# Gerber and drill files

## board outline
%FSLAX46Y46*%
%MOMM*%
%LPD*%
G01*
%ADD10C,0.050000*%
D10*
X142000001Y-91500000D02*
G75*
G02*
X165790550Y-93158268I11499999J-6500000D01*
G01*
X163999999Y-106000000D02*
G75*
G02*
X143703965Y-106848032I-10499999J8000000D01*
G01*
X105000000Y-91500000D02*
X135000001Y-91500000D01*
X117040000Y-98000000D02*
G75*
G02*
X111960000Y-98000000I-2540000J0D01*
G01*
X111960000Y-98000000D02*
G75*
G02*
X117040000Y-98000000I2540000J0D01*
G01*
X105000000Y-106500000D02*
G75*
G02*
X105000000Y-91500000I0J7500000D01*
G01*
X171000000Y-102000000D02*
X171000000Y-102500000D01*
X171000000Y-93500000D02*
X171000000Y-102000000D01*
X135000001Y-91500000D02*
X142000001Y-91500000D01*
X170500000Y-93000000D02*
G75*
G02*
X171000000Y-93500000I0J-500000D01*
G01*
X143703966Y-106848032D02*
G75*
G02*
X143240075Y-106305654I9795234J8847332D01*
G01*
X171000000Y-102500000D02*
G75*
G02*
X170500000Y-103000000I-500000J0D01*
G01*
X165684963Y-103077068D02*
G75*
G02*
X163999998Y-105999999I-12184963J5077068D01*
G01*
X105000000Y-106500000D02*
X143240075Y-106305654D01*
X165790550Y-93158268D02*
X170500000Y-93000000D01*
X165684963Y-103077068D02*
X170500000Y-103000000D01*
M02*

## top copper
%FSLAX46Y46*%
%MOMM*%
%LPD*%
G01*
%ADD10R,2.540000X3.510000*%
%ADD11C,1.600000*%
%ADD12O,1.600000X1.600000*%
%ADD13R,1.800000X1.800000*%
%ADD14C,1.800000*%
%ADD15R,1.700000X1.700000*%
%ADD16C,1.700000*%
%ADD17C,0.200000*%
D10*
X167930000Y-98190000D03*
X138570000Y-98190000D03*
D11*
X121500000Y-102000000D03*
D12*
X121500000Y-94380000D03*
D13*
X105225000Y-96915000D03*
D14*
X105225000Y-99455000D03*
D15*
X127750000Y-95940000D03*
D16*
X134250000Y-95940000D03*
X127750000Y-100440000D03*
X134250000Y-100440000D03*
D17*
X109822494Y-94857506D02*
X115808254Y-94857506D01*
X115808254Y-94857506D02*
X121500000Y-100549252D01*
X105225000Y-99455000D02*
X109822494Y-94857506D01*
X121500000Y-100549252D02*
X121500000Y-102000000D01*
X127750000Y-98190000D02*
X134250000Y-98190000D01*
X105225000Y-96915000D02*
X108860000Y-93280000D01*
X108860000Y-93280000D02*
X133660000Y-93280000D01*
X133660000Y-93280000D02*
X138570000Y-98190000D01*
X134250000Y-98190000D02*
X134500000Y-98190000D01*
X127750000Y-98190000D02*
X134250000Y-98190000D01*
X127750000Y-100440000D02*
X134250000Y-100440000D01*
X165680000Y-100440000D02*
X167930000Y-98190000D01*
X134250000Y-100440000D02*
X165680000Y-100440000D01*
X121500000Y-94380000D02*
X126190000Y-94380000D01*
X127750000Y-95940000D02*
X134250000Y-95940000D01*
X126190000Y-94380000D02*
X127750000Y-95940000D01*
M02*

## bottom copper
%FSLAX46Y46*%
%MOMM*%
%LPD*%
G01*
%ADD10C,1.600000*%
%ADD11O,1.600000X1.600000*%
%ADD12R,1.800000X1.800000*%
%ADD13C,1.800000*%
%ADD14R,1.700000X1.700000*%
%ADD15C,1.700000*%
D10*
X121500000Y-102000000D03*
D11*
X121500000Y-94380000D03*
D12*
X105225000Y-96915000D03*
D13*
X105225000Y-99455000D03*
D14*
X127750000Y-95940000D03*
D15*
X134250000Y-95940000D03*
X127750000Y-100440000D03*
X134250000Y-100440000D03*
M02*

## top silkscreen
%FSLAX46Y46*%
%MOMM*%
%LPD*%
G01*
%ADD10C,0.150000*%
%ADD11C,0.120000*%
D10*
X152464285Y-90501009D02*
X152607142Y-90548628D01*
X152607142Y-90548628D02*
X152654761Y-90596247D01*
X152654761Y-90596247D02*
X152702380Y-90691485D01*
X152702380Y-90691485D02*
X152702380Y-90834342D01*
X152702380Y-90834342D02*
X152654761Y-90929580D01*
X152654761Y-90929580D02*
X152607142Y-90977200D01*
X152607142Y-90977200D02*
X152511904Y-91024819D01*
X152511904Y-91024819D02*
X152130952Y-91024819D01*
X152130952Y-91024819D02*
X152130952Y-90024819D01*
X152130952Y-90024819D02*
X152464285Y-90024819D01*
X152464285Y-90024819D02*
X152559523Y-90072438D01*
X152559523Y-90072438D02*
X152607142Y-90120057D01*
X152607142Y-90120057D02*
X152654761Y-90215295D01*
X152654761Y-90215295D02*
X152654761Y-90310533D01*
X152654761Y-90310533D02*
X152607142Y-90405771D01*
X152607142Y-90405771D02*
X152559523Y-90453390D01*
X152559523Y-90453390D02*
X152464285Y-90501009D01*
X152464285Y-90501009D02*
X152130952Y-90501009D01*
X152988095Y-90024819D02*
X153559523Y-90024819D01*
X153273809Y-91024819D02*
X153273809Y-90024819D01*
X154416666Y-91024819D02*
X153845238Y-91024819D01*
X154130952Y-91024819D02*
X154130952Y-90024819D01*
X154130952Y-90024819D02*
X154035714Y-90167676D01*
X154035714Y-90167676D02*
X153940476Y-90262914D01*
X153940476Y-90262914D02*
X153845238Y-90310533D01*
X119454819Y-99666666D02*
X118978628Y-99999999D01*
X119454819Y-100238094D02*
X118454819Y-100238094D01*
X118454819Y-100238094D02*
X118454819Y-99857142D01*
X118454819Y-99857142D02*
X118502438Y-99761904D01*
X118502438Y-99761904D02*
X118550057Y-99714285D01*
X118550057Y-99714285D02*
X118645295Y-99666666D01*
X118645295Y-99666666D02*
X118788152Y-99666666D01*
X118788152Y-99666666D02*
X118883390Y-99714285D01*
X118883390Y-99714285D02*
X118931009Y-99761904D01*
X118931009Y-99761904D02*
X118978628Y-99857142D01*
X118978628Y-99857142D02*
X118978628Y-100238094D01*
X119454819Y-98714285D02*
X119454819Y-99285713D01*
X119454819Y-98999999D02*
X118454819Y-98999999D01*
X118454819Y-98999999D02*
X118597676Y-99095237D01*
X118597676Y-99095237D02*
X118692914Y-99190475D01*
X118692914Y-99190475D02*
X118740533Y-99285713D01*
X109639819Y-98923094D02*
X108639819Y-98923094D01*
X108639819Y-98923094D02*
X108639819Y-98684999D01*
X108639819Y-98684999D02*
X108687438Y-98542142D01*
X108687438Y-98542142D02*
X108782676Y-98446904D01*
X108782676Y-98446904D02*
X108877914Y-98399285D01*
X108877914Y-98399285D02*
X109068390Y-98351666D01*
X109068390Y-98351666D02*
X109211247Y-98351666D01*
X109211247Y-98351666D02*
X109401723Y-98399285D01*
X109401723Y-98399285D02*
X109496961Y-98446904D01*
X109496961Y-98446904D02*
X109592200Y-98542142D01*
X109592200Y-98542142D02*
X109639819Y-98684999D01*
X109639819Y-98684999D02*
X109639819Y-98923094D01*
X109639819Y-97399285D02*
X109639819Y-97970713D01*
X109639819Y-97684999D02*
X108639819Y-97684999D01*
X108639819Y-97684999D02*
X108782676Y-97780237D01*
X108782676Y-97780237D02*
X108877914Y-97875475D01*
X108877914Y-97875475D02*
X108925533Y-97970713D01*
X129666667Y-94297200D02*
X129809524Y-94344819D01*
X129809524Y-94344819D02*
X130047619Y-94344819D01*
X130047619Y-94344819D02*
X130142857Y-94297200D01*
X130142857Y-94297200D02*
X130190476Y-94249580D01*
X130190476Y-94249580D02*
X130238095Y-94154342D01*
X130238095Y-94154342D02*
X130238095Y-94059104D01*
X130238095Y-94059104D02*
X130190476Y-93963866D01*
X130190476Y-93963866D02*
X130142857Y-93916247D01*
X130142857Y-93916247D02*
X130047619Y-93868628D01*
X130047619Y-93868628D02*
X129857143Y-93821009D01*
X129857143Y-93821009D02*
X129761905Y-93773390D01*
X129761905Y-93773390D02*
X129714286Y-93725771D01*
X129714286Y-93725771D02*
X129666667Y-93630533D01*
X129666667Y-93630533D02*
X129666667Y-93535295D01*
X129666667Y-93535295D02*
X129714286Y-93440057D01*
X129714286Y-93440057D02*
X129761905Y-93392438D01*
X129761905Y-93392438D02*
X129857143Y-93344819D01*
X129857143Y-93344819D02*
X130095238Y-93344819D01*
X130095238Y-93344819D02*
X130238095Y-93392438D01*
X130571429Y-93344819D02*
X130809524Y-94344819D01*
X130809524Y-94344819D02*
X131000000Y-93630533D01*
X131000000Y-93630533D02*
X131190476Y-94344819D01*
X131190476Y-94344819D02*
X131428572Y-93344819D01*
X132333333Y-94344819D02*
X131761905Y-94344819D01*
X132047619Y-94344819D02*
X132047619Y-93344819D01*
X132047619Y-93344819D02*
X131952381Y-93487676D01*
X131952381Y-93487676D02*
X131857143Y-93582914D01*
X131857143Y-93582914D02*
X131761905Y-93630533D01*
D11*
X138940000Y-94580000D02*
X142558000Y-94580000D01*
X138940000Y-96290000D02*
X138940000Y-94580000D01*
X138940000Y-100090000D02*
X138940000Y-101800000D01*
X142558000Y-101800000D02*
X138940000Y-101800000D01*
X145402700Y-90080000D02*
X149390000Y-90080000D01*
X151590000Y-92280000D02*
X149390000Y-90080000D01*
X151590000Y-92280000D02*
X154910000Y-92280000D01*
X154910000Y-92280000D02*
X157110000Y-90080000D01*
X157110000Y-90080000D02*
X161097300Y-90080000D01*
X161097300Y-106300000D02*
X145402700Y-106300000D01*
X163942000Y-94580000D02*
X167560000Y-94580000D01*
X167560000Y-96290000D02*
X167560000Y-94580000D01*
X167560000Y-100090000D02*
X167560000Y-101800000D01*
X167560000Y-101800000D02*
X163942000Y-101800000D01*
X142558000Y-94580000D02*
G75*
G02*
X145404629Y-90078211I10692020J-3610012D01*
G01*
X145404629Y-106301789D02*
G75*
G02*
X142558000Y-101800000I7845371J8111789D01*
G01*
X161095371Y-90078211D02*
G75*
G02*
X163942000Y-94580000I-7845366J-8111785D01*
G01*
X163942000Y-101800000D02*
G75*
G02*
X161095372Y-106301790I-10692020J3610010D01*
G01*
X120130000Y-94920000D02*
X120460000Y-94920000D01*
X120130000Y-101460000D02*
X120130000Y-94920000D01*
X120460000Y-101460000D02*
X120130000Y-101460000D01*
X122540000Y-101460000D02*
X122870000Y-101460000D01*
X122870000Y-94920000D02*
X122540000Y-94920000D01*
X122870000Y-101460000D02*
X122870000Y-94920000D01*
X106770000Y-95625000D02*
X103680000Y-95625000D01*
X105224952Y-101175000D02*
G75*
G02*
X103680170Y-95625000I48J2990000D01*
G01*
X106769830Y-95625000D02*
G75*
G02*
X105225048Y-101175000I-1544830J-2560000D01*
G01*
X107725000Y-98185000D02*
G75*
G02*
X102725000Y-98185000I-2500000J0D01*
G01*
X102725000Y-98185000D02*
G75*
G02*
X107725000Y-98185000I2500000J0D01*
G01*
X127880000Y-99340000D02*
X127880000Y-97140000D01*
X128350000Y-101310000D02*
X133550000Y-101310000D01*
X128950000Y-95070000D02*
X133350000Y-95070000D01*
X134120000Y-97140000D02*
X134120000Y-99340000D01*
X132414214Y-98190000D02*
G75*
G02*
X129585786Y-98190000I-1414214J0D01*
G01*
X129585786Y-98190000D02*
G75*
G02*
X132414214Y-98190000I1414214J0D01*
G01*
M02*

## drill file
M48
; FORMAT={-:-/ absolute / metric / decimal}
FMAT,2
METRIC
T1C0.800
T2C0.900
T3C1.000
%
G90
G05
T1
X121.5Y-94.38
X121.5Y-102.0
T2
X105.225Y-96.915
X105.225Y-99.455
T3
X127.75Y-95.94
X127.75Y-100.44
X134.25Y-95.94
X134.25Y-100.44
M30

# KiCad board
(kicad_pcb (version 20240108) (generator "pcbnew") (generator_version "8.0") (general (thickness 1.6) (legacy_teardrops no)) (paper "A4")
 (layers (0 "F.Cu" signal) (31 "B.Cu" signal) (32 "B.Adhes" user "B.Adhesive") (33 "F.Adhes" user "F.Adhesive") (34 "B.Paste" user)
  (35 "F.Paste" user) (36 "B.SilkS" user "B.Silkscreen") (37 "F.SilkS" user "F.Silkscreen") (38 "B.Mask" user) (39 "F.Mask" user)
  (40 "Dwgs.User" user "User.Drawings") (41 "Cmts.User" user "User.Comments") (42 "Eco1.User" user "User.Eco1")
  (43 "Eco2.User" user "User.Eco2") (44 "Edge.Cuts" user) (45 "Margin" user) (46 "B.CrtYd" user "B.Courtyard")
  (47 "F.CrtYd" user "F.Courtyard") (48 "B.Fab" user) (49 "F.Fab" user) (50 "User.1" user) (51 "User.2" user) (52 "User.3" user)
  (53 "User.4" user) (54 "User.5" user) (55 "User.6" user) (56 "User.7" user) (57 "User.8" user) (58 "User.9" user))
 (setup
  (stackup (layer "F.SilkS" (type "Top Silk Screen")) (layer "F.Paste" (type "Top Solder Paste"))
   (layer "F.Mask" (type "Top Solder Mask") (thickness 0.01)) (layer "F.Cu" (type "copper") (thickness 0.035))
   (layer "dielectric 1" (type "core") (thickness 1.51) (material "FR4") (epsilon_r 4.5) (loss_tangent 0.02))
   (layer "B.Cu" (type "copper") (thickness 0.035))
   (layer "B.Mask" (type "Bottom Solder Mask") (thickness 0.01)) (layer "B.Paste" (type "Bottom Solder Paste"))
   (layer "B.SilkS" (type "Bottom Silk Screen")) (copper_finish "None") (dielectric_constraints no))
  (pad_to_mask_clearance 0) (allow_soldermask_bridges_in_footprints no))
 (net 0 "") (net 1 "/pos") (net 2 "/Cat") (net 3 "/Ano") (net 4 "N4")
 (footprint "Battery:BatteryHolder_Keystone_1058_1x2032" (layer "F.Cu") (at 153.25 98.19 180)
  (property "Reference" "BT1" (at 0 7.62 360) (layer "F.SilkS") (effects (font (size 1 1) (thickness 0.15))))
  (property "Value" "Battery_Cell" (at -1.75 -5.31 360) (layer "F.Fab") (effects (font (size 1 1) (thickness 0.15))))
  (fp_line (start 14.31 3.61) (end 10.692 3.61) (stroke (width 0.12) (type solid)) (layer "F.SilkS"))
  (fp_line (start 14.31 1.9) (end 14.31 3.61) (stroke (width 0.12) (type solid)) (layer "F.SilkS"))
  (fp_line (start 14.31 -1.9) (end 14.31 -3.61) (stroke (width 0.12) (type solid)) (layer "F.SilkS"))
  (fp_line (start 10.692 -3.61) (end 14.31 -3.61) (stroke (width 0.12) (type solid)) (layer "F.SilkS"))
  (fp_line (start 7.8473 8.11) (end 3.86 8.11) (stroke (width 0.12) (type solid)) (layer "F.SilkS"))
  (fp_line (start 1.66 5.91) (end 3.86 8.11) (stroke (width 0.12) (type solid)) (layer "F.SilkS"))
  (fp_line (start 1.66 5.91) (end -1.66 5.91) (stroke (width 0.12) (type solid)) (layer "F.SilkS"))
  (fp_line (start -1.66 5.91) (end -3.86 8.11) (stroke (width 0.12) (type solid)) (layer "F.SilkS"))
  (fp_line (start -3.86 8.11) (end -7.8473 8.11) (stroke (width 0.12) (type solid)) (layer "F.SilkS"))
  (fp_line (start -7.8473 -8.11) (end 7.8473 -8.11) (stroke (width 0.12) (type solid)) (layer "F.SilkS"))
  (fp_line (start -10.692 3.61) (end -14.31 3.61) (stroke (width 0.12) (type solid)) (layer "F.SilkS"))
  (fp_line (start -14.31 1.9) (end -14.31 3.61) (stroke (width 0.12) (type solid)) (layer "F.SilkS"))
  (fp_line (start -14.31 -1.9) (end -14.31 -3.61) (stroke (width 0.12) (type solid)) (layer "F.SilkS"))
  (fp_line (start -14.31 -3.61) (end -10.692 -3.61) (stroke (width 0.12) (type solid)) (layer "F.SilkS"))
  (fp_arc (start 10.692 3.61) (mid 9.538084 6.031244) (end 7.845371 8.111789) (stroke (width 0.12) (type solid)) (layer "F.SilkS"))
  (fp_arc (start 7.845371 -8.111789) (mid 9.538085 -6.031244) (end 10.692 -3.61) (stroke (width 0.12) (type solid)) (layer "F.SilkS"))
  (fp_arc (start -7.845371 8.111789) (mid -9.538085 6.031244) (end -10.692 3.61) (stroke (width 0.12) (type solid)) (layer "F.SilkS"))
  (fp_arc (start -10.692 -3.61) (mid -9.538084 -6.031244) (end -7.845371 -8.111789) (stroke (width 0.12) (type solid)) (layer "F.SilkS"))
  (pad "1" smd rect (at -14.68 0 180) (size 2.54 3.51) (layers "F.Cu" "F.Paste" "F.Mask") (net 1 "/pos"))
  (pad "2" smd rect (at 14.68 0 180) (size 2.54 3.51) (layers "F.Cu" "F.Paste" "F.Mask") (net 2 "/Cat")))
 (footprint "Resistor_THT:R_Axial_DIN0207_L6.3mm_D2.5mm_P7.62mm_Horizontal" (layer "F.Cu") (at 121.5 102 90)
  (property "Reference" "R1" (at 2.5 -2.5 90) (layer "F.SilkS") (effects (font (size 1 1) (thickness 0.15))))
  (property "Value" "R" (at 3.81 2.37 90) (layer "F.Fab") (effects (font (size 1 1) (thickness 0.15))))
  (fp_line (start 7.08 -1.37) (end 7.08 -1.04) (stroke (width 0.12) (type solid)) (layer "F.SilkS"))
  (fp_line (start 0.54 -1.37) (end 7.08 -1.37) (stroke (width 0.12) (type solid)) (layer "F.SilkS"))
  (fp_line (start 0.54 -1.04) (end 0.54 -1.37) (stroke (width 0.12) (type solid)) (layer "F.SilkS"))
  (fp_line (start 0.54 1.04) (end 0.54 1.37) (stroke (width 0.12) (type solid)) (layer "F.SilkS"))
  (fp_line (start 7.08 1.37) (end 7.08 1.04) (stroke (width 0.12) (type solid)) (layer "F.SilkS"))
  (fp_line (start 0.54 1.37) (end 7.08 1.37) (stroke (width 0.12) (type solid)) (layer "F.SilkS"))
  (pad "1" thru_hole circle (at 0 0 90) (size 1.6 1.6) (drill 0.8) (layers "*.Cu" "*.Mask") (remove_unused_layers no) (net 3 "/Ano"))
  (pad "2" thru_hole oval (at 7.62 0 90) (size 1.6 1.6) (drill 0.8) (layers "*.Cu" "*.Mask") (remove_unused_layers no) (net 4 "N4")))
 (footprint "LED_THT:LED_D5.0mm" (layer "F.Cu") (at 105.225 96.915 -90)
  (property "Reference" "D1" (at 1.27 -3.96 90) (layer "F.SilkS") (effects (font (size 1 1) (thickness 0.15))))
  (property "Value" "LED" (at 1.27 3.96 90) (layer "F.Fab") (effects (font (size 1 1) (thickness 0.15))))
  (fp_line (start -1.29 -1.545) (end -1.29 1.545) (stroke (width 0.12) (type solid)) (layer "F.SilkS"))
  (fp_arc (start 4.26 0.000048) (mid 2.071756 2.880501) (end -1.29 1.54483) (stroke (width 0.12) (type solid)) (layer "F.SilkS"))
  (fp_arc (start -1.29 -1.54483) (mid 2.071756 -2.880501) (end 4.26 -0.000048) (stroke (width 0.12) (type solid)) (layer "F.SilkS"))
  (fp_circle (center 1.27 0) (end 3.77 0) (stroke (width 0.12) (type solid)) (fill none) (layer "F.SilkS"))
  (pad "1" thru_hole rect (at 0 0 270) (size 1.8 1.8) (drill 0.9) (layers "*.Cu" "*.Mask") (remove_unused_layers no) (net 2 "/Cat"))
  (pad "2" thru_hole circle (at 2.54 0 270) (size 1.8 1.8) (drill 0.9) (layers "*.Cu" "*.Mask") (remove_unused_layers no) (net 3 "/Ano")))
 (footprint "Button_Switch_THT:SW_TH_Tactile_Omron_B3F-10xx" (layer "F.Cu") (at 127.75 95.94)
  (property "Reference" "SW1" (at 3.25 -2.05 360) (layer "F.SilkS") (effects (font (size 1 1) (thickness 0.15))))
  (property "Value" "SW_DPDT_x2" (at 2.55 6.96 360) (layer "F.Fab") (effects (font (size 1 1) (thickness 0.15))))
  (fp_line (start 0.13 3.4) (end 0.13 1.2) (stroke (width 0.12) (type solid)) (layer "F.SilkS"))
  (fp_line (start 0.6 5.37) (end 5.8 5.37) (stroke (width 0.12) (type solid)) (layer "F.SilkS"))
  (fp_line (start 1.2 -0.87) (end 5.6 -0.87) (stroke (width 0.12) (type solid)) (layer "F.SilkS"))
  (fp_line (start 6.37 1.2) (end 6.37 3.4) (stroke (width 0.12) (type solid)) (layer "F.SilkS"))
  (fp_circle (center 3.25 2.25) (end 4.25 3.25) (stroke (width 0.12) (type solid)) (fill none) (layer "F.SilkS"))
  (pad "1" thru_hole rect (at 0 0) (size 1.7 1.7) (drill 1) (layers "*.Cu" "*.Mask") (remove_unused_layers no) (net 4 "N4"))
  (pad "1" thru_hole circle (at 6.5 0) (size 1.7 1.7) (drill 1) (layers "*.Cu" "*.Mask") (remove_unused_layers no) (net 4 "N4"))
  (pad "2" thru_hole circle (at 0 4.5) (size 1.7 1.7) (drill 1) (layers "*.Cu" "*.Mask") (remove_unused_layers no) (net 1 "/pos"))
  (pad "2" thru_hole circle (at 6.5 4.5) (size 1.7 1.7) (drill 1) (layers "*.Cu" "*.Mask") (remove_unused_layers no) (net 1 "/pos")))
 (gr_arc (start 142.000001 91.5) (mid 154.418535 84.822129) (end 165.79055 93.158268) (locked yes) (stroke (width 0.05) (type default))
  (layer "Edge.Cuts"))
 (gr_arc (start 163.999999 106) (mid 154.051073 111.18887) (end 143.703965 106.848032) (locked yes) (stroke (width 0.05) (type default))
  (layer "Edge.Cuts"))
 (gr_line (start 105 91.5) (end 135.000001 91.5) (locked yes) (stroke (width 0.05) (type default)) (layer "Edge.Cuts"))
 (gr_circle (center 114.5 98) (end 114.5 100.54) (stroke (width 0.05) (type default)) (fill none) (layer "Edge.Cuts"))
 (gr_arc (start 105 106.5) (mid 97.5 99) (end 105 91.5) (locked yes) (stroke (width 0.05) (type default)) (layer "Edge.Cuts"))
 (gr_line (start 171 102) (end 171 102.5) (locked yes) (stroke (width 0.05) (type default)) (layer "Edge.Cuts"))
 (gr_line (start 171 93.5) (end 171 102) (locked yes) (stroke (width 0.05) (type default)) (layer "Edge.Cuts"))
 (gr_line (start 135.000001 91.5) (end 142.000001 91.5) (locked yes) (stroke (width 0.05) (type default)) (layer "Edge.Cuts"))
 (gr_arc (start 170.5 93) (mid 170.853553 93.146447) (end 171 93.5) (locked yes) (stroke (width 0.05) (type default)) (layer "Edge.Cuts"))
 (gr_arc (start 143.703966 106.848032) (mid 143.468354 106.579979) (end 143.240075 106.305654) (locked yes)
  (stroke (width 0.05) (type default)) (layer "Edge.Cuts"))
 (gr_arc (start 171 102.5) (mid 170.853553 102.853553) (end 170.5 103) (locked yes) (stroke (width 0.05) (type default)) (layer "Edge.Cuts"))
 (gr_arc (start 165.684963 103.077068) (mid 164.936247 104.592587) (end 163.999998 105.999999) (locked yes)
  (stroke (width 0.05) (type default)) (layer "Edge.Cuts"))
 (gr_line (start 105 106.5) (end 143.240075 106.305654) (locked yes) (stroke (width 0.05) (type default)) (layer "Edge.Cuts"))
 (gr_line (start 165.79055 93.158268) (end 170.5 93) (locked yes) (stroke (width 0.05) (type default)) (layer "Edge.Cuts"))
 (gr_line (start 165.684963 103.077068) (end 170.5 103) (locked yes) (stroke (width 0.05) (type default)) (layer "Edge.Cuts"))
 (segment (start 109.822494 94.857506) (end 115.808254 94.857506) (width 0.2) (layer "F.Cu") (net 3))
 (segment (start 115.808254 94.857506) (end 121.5 100.549252) (width 0.2) (layer "F.Cu") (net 3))
 (segment (start 105.225 99.455) (end 109.822494 94.857506) (width 0.2) (layer "F.Cu") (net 3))
 (segment (start 121.5 100.549252) (end 121.5 102) (width 0.2) (layer "F.Cu") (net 3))
 (segment (start 127.75 98.19) (end 134.25 98.19) (width 0.2) (layer "F.Cu") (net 2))
 (segment (start 105.225 96.915) (end 108.86 93.28) (width 0.2) (layer "F.Cu") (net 2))
 (segment (start 108.86 93.28) (end 133.66 93.28) (width 0.2) (layer "F.Cu") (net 2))
 (segment (start 133.66 93.28) (end 138.57 98.19) (width 0.2) (layer "F.Cu") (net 2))
 (segment (start 134.25 98.19) (end 134.5 98.19) (width 0.2) (layer "F.Cu") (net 2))
 (segment (start 127.75 98.19) (end 134.25 98.19) (width 0.2) (layer "F.Cu") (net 2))
 (segment (start 127.75 100.44) (end 134.25 100.44) (width 0.2) (layer "F.Cu") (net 1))
 (segment (start 165.68 100.44) (end 167.93 98.19) (width 0.2) (layer "F.Cu") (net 1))
 (segment (start 134.25 100.44) (end 165.68 100.44) (width 0.2) (layer "F.Cu") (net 1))
 (segment (start 121.5 94.38) (end 126.19 94.38) (width 0.2) (layer "F.Cu") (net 4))
 (segment (start 127.75 95.94) (end 134.25 95.94) (width 0.2) (layer "F.Cu") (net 4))
 (segment (start 126.19 94.38) (end 127.75 95.94) (width 0.2) (layer "F.Cu") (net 4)))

